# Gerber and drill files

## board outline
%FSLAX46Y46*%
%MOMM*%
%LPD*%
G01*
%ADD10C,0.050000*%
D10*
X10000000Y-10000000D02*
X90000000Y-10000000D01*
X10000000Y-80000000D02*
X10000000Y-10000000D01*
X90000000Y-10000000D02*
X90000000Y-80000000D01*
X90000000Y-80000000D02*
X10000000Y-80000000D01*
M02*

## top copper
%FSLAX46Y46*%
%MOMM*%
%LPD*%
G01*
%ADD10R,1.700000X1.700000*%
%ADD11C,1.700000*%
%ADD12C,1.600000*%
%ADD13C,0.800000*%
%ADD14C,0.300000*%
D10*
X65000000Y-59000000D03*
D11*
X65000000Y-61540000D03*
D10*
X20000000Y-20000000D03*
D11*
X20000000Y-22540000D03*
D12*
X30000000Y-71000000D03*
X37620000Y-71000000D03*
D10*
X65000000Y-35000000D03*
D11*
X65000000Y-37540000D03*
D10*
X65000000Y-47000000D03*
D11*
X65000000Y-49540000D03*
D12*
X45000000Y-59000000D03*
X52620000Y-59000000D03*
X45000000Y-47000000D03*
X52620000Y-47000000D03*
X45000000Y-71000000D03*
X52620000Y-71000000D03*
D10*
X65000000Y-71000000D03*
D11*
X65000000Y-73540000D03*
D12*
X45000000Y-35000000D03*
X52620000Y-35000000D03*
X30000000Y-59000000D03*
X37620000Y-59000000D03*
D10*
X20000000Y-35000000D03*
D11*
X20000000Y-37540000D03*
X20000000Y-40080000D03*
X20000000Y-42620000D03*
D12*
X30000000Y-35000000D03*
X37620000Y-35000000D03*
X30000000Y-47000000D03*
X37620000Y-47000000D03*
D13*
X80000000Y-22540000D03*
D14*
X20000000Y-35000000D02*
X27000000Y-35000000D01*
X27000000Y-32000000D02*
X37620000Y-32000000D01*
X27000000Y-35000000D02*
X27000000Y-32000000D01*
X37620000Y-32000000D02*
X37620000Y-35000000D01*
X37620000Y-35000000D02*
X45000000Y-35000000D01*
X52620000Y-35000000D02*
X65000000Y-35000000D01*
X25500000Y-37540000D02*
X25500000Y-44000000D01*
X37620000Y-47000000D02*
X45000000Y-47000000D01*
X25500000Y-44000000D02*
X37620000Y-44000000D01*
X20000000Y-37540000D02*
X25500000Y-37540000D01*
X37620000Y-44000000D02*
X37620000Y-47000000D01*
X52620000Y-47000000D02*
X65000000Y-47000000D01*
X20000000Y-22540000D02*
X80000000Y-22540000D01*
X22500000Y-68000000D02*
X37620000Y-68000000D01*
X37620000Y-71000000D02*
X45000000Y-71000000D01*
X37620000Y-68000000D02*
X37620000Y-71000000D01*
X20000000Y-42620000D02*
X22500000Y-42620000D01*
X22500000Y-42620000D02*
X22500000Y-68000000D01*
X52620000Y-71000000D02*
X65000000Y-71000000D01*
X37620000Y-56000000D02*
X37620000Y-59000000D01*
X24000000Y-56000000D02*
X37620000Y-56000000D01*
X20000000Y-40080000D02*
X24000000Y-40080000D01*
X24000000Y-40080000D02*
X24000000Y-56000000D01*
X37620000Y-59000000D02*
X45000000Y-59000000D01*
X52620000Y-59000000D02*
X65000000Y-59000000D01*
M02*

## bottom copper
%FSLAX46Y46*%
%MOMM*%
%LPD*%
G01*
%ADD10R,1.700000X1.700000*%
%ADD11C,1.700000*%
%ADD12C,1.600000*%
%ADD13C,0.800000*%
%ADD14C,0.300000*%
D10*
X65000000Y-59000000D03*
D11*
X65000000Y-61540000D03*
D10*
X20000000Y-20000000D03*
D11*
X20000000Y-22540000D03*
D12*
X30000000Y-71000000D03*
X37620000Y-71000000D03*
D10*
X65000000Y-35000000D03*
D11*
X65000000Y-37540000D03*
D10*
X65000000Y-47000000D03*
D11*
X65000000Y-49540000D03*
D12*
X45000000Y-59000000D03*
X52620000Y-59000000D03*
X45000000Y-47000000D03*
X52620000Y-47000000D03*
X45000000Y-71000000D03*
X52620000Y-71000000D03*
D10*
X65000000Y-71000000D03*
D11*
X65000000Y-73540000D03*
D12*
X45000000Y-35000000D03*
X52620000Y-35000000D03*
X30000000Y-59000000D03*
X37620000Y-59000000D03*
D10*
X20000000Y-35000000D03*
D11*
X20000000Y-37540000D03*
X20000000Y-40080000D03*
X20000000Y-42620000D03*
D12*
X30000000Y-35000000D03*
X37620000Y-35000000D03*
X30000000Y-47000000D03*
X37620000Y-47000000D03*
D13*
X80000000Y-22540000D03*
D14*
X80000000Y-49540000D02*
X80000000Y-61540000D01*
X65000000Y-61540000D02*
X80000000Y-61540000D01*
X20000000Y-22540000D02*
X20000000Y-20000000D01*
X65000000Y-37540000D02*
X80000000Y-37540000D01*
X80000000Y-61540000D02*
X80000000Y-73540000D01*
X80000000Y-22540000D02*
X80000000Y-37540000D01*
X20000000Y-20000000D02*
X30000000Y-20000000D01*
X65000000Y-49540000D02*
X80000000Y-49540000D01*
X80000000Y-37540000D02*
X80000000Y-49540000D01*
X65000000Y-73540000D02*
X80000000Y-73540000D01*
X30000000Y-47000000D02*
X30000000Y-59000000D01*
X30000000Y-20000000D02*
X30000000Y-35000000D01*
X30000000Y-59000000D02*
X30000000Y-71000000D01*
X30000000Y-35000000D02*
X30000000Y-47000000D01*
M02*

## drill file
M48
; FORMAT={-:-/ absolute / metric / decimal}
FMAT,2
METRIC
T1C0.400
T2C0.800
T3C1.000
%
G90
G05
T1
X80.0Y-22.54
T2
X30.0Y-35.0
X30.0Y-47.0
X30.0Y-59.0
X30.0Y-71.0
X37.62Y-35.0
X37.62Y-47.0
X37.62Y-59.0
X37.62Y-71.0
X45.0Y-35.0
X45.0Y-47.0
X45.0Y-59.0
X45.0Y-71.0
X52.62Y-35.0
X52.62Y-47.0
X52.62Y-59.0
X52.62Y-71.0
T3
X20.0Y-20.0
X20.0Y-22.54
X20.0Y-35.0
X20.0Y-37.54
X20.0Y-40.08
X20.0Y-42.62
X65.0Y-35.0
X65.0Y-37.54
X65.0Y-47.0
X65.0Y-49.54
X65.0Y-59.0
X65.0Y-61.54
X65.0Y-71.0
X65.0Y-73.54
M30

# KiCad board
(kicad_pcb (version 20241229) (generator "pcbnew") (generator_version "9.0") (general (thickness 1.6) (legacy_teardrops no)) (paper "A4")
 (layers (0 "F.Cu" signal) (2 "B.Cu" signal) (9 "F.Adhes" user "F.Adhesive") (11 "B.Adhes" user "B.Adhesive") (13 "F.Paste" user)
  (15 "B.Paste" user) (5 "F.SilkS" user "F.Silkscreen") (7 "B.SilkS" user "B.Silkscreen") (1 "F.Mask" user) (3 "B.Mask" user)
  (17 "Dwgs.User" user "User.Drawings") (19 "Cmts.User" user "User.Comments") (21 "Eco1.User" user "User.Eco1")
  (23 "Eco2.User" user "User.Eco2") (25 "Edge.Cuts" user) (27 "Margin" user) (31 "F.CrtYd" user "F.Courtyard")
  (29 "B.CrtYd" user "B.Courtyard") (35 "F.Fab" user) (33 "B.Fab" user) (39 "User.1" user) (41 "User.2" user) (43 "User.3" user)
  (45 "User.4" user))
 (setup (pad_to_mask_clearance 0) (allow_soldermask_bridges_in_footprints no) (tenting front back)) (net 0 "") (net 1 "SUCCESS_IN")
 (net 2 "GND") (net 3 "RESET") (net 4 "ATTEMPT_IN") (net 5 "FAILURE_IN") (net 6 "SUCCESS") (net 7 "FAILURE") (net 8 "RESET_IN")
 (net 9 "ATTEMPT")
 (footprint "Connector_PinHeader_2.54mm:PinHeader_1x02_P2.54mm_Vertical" (layer "F.Cu") (at 65 59)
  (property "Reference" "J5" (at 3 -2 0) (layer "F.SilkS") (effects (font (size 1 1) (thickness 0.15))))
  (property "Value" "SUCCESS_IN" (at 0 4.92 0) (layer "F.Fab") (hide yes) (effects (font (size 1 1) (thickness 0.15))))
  (pad "1" thru_hole rect (at 0 0) (size 1.7 1.7) (drill 1) (layers "*.Cu" "*.Mask") (remove_unused_layers no) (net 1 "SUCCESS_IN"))
  (pad "2" thru_hole circle (at 0 2.54) (size 1.7 1.7) (drill 1) (layers "*.Cu" "*.Mask") (remove_unused_layers no) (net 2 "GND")))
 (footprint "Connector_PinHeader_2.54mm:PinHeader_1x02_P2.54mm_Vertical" (layer "F.Cu") (at 20 20)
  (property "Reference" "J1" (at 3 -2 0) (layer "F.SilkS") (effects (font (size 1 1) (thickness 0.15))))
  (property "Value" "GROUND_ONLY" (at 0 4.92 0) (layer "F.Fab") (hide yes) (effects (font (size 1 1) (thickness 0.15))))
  (pad "1" thru_hole rect (at 0 0) (size 1.7 1.7) (drill 1) (layers "*.Cu" "*.Mask") (remove_unused_layers no) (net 2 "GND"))
  (pad "2" thru_hole circle (at 0 2.54) (size 1.7 1.7) (drill 1) (layers "*.Cu" "*.Mask") (remove_unused_layers no) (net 2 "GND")))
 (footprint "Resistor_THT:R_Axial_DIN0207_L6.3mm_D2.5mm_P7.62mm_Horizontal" (layer "F.Cu") (at 30 71)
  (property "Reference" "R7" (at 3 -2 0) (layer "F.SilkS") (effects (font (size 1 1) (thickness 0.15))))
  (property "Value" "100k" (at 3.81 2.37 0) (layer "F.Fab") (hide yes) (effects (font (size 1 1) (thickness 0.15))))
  (pad "1" thru_hole circle (at 0 0) (size 1.6 1.6) (drill 0.8) (layers "*.Cu" "*.Mask") (remove_unused_layers no) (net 2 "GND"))
  (pad "2" thru_hole circle (at 7.62 0) (size 1.6 1.6) (drill 0.8) (layers "*.Cu" "*.Mask") (remove_unused_layers no) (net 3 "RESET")))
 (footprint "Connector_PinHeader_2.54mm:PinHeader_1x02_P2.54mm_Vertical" (layer "F.Cu") (at 65 35)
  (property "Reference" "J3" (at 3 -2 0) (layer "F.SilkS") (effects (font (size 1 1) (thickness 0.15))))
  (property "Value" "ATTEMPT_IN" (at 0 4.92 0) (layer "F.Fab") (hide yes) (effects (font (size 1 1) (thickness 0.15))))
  (pad "1" thru_hole rect (at 0 0) (size 1.7 1.7) (drill 1) (layers "*.Cu" "*.Mask") (remove_unused_layers no) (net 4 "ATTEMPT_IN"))
  (pad "2" thru_hole circle (at 0 2.54) (size 1.7 1.7) (drill 1) (layers "*.Cu" "*.Mask") (remove_unused_layers no) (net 2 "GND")))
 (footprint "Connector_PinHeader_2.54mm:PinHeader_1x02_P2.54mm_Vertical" (layer "F.Cu") (at 65 47)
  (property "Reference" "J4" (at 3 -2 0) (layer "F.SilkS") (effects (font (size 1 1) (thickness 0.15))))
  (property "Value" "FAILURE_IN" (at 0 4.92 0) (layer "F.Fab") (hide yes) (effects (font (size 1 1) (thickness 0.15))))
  (pad "1" thru_hole rect (at 0 0) (size 1.7 1.7) (drill 1) (layers "*.Cu" "*.Mask") (remove_unused_layers no) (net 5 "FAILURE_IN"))
  (pad "2" thru_hole circle (at 0 2.54) (size 1.7 1.7) (drill 1) (layers "*.Cu" "*.Mask") (remove_unused_layers no) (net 2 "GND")))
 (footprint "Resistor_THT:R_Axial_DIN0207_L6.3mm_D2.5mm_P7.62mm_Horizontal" (layer "F.Cu") (at 45 59)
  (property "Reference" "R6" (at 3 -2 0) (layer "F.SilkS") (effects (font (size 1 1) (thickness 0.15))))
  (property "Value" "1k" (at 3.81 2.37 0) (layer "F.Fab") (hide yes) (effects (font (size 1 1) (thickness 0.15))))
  (pad "1" thru_hole circle (at 0 0) (size 1.6 1.6) (drill 0.8) (layers "*.Cu" "*.Mask") (remove_unused_layers no) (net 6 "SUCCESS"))
  (pad "2" thru_hole circle (at 7.62 0) (size 1.6 1.6) (drill 0.8) (layers "*.Cu" "*.Mask") (remove_unused_layers no) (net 1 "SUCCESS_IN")))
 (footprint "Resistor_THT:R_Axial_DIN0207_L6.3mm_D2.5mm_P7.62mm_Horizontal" (layer "F.Cu") (at 45 47)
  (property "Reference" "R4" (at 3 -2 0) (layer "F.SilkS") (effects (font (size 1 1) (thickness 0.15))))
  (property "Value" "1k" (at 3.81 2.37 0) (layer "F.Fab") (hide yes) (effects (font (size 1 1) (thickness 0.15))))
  (pad "1" thru_hole circle (at 0 0) (size 1.6 1.6) (drill 0.8) (layers "*.Cu" "*.Mask") (remove_unused_layers no) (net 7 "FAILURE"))
  (pad "2" thru_hole circle (at 7.62 0) (size 1.6 1.6) (drill 0.8) (layers "*.Cu" "*.Mask") (remove_unused_layers no) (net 5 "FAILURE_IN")))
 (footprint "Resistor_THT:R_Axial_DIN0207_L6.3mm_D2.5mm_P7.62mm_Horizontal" (layer "F.Cu") (at 45 71)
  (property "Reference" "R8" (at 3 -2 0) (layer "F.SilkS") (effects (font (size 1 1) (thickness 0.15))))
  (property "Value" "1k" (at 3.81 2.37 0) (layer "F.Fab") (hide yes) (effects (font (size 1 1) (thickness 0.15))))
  (pad "1" thru_hole circle (at 0 0) (size 1.6 1.6) (drill 0.8) (layers "*.Cu" "*.Mask") (remove_unused_layers no) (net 3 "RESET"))
  (pad "2" thru_hole circle (at 7.62 0) (size 1.6 1.6) (drill 0.8) (layers "*.Cu" "*.Mask") (remove_unused_layers no) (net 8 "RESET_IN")))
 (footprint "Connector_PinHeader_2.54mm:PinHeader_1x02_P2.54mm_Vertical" (layer "F.Cu") (at 65 71)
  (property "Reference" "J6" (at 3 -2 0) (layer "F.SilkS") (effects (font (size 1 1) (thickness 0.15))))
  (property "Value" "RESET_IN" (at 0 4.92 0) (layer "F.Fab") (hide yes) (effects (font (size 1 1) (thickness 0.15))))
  (pad "1" thru_hole rect (at 0 0) (size 1.7 1.7) (drill 1) (layers "*.Cu" "*.Mask") (remove_unused_layers no) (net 8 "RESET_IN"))
  (pad "2" thru_hole circle (at 0 2.54) (size 1.7 1.7) (drill 1) (layers "*.Cu" "*.Mask") (remove_unused_layers no) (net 2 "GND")))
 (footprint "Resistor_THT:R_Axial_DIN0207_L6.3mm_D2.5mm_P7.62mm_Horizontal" (layer "F.Cu") (at 45 35)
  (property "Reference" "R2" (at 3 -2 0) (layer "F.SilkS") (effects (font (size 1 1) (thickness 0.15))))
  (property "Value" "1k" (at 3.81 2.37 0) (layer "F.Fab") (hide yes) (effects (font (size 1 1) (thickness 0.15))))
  (pad "1" thru_hole circle (at 0 0) (size 1.6 1.6) (drill 0.8) (layers "*.Cu" "*.Mask") (remove_unused_layers no) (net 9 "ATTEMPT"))
  (pad "2" thru_hole circle (at 7.62 0) (size 1.6 1.6) (drill 0.8) (layers "*.Cu" "*.Mask") (remove_unused_layers no) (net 4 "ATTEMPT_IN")))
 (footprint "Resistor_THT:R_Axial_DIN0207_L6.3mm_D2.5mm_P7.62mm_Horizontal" (layer "F.Cu") (at 30 59)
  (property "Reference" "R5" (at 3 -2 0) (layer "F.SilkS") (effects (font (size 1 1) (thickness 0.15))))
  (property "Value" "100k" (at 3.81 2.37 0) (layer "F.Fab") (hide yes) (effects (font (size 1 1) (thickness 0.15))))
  (pad "1" thru_hole circle (at 0 0) (size 1.6 1.6) (drill 0.8) (layers "*.Cu" "*.Mask") (remove_unused_layers no) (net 2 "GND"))
  (pad "2" thru_hole circle (at 7.62 0) (size 1.6 1.6) (drill 0.8) (layers "*.Cu" "*.Mask") (remove_unused_layers no) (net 6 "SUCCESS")))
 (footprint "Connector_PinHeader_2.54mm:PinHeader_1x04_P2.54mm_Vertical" (layer "F.Cu") (at 20 35)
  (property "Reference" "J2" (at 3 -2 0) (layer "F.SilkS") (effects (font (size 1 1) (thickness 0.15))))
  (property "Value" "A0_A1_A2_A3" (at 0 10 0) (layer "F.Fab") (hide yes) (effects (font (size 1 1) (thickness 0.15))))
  (pad "1" thru_hole rect (at 0 0) (size 1.7 1.7) (drill 1) (layers "*.Cu" "*.Mask") (remove_unused_layers no) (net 9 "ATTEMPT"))
  (pad "2" thru_hole circle (at 0 2.54) (size 1.7 1.7) (drill 1) (layers "*.Cu" "*.Mask") (remove_unused_layers no) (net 7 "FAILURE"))
  (pad "3" thru_hole circle (at 0 5.08) (size 1.7 1.7) (drill 1) (layers "*.Cu" "*.Mask") (remove_unused_layers no) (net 6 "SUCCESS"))
  (pad "4" thru_hole circle (at 0 7.62) (size 1.7 1.7) (drill 1) (layers "*.Cu" "*.Mask") (remove_unused_layers no) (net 3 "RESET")))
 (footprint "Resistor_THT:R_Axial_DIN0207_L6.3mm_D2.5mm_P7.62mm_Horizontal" (layer "F.Cu") (at 30 35)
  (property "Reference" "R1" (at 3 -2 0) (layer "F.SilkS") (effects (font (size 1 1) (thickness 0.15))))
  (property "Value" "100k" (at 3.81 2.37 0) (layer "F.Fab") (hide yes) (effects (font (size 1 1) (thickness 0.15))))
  (pad "1" thru_hole circle (at 0 0) (size 1.6 1.6) (drill 0.8) (layers "*.Cu" "*.Mask") (remove_unused_layers no) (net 2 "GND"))
  (pad "2" thru_hole circle (at 7.62 0) (size 1.6 1.6) (drill 0.8) (layers "*.Cu" "*.Mask") (remove_unused_layers no) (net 9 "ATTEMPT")))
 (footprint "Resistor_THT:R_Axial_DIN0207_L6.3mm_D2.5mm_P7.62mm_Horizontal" (layer "F.Cu") (at 30 47)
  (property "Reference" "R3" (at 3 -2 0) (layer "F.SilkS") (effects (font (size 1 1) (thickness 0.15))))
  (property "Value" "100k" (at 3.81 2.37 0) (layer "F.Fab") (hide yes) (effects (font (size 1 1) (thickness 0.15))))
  (pad "1" thru_hole circle (at 0 0) (size 1.6 1.6) (drill 0.8) (layers "*.Cu" "*.Mask") (remove_unused_layers no) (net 2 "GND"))
  (pad "2" thru_hole circle (at 7.62 0) (size 1.6 1.6) (drill 0.8) (layers "*.Cu" "*.Mask") (remove_unused_layers no) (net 7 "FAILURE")))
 (gr_line (start 10 10) (end 90 10) (stroke (width 0.05) (type default)) (layer "Edge.Cuts"))
 (gr_line (start 10 80) (end 10 10) (stroke (width 0.05) (type default)) (layer "Edge.Cuts"))
 (gr_line (start 90 10) (end 90 80) (stroke (width 0.05) (type default)) (layer "Edge.Cuts"))
 (gr_line (start 90 80) (end 10 80) (stroke (width 0.05) (type default)) (layer "Edge.Cuts"))
 (segment (start 20 35) (end 27 35) (width 0.3) (layer "F.Cu") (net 9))
 (segment (start 27 32) (end 37.62 32) (width 0.3) (layer "F.Cu") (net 9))
 (segment (start 27 35) (end 27 32) (width 0.3) (layer "F.Cu") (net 9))
 (segment (start 37.62 32) (end 37.62 35) (width 0.3) (layer "F.Cu") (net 9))
 (segment (start 37.62 35) (end 45 35) (width 0.3) (layer "F.Cu") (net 9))
 (segment (start 52.62 35) (end 65 35) (width 0.3) (layer "F.Cu") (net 4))
 (segment (start 25.5 37.54) (end 25.5 44) (width 0.3) (layer "F.Cu") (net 7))
 (segment (start 37.62 47) (end 45 47) (width 0.3) (layer "F.Cu") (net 7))
 (segment (start 25.5 44) (end 37.62 44) (width 0.3) (layer "F.Cu") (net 7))
 (segment (start 20 37.54) (end 25.5 37.54) (width 0.3) (layer "F.Cu") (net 7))
 (segment (start 37.62 44) (end 37.62 47) (width 0.3) (layer "F.Cu") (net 7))
 (segment (start 52.62 47) (end 65 47) (width 0.3) (layer "F.Cu") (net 5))
 (segment (start 20 22.54) (end 80 22.54) (width 0.3) (layer "F.Cu") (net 2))
 (via (at 80 22.54) (size 0.8) (drill 0.4) (layers "F.Cu" "B.Cu") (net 2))
 (segment (start 80 49.54) (end 80 61.54) (width 0.3) (layer "B.Cu") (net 2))
 (segment (start 65 61.54) (end 80 61.54) (width 0.3) (layer "B.Cu") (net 2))
 (segment (start 20 22.54) (end 20 20) (width 0.3) (layer "B.Cu") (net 2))
 (segment (start 65 37.54) (end 80 37.54) (width 0.3) (layer "B.Cu") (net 2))
 (segment (start 80 61.54) (end 80 73.54) (width 0.3) (layer "B.Cu") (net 2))
 (segment (start 80 22.54) (end 80 37.54) (width 0.3) (layer "B.Cu") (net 2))
 (segment (start 20 20) (end 30 20) (width 0.3) (layer "B.Cu") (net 2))
 (segment (start 65 49.54) (end 80 49.54) (width 0.3) (layer "B.Cu") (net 2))
 (segment (start 80 37.54) (end 80 49.54) (width 0.3) (layer "B.Cu") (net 2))
 (segment (start 65 73.54) (end 80 73.54) (width 0.3) (layer "B.Cu") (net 2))
 (segment (start 30 47) (end 30 59) (width 0.3) (layer "B.Cu") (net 2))
 (segment (start 30 20) (end 30 35) (width 0.3) (layer "B.Cu") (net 2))
 (segment (start 30 59) (end 30 71) (width 0.3) (layer "B.Cu") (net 2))
 (segment (start 30 35) (end 30 47) (width 0.3) (layer "B.Cu") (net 2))
 (segment (start 22.5 68) (end 37.62 68) (width 0.3) (layer "F.Cu") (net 3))
 (segment (start 37.62 71) (end 45 71) (width 0.3) (layer "F.Cu") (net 3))
 (segment (start 37.62 68) (end 37.62 71) (width 0.3) (layer "F.Cu") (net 3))
 (segment (start 20 42.62) (end 22.5 42.62) (width 0.3) (layer "F.Cu") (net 3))
 (segment (start 22.5 42.62) (end 22.5 68) (width 0.3) (layer "F.Cu") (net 3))
 (segment (start 52.62 71) (end 65 71) (width 0.3) (layer "F.Cu") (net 8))
 (segment (start 37.62 56) (end 37.62 59) (width 0.3) (layer "F.Cu") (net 6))
 (segment (start 24 56) (end 37.62 56) (width 0.3) (layer "F.Cu") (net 6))
 (segment (start 20 40.08) (end 24 40.08) (width 0.3) (layer "F.Cu") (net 6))
 (segment (start 24 40.08) (end 24 56) (width 0.3) (layer "F.Cu") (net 6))
 (segment (start 37.62 59) (end 45 59) (width 0.3) (layer "F.Cu") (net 6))
 (segment (start 52.62 59) (end 65 59) (width 0.3) (layer "F.Cu") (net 1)))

